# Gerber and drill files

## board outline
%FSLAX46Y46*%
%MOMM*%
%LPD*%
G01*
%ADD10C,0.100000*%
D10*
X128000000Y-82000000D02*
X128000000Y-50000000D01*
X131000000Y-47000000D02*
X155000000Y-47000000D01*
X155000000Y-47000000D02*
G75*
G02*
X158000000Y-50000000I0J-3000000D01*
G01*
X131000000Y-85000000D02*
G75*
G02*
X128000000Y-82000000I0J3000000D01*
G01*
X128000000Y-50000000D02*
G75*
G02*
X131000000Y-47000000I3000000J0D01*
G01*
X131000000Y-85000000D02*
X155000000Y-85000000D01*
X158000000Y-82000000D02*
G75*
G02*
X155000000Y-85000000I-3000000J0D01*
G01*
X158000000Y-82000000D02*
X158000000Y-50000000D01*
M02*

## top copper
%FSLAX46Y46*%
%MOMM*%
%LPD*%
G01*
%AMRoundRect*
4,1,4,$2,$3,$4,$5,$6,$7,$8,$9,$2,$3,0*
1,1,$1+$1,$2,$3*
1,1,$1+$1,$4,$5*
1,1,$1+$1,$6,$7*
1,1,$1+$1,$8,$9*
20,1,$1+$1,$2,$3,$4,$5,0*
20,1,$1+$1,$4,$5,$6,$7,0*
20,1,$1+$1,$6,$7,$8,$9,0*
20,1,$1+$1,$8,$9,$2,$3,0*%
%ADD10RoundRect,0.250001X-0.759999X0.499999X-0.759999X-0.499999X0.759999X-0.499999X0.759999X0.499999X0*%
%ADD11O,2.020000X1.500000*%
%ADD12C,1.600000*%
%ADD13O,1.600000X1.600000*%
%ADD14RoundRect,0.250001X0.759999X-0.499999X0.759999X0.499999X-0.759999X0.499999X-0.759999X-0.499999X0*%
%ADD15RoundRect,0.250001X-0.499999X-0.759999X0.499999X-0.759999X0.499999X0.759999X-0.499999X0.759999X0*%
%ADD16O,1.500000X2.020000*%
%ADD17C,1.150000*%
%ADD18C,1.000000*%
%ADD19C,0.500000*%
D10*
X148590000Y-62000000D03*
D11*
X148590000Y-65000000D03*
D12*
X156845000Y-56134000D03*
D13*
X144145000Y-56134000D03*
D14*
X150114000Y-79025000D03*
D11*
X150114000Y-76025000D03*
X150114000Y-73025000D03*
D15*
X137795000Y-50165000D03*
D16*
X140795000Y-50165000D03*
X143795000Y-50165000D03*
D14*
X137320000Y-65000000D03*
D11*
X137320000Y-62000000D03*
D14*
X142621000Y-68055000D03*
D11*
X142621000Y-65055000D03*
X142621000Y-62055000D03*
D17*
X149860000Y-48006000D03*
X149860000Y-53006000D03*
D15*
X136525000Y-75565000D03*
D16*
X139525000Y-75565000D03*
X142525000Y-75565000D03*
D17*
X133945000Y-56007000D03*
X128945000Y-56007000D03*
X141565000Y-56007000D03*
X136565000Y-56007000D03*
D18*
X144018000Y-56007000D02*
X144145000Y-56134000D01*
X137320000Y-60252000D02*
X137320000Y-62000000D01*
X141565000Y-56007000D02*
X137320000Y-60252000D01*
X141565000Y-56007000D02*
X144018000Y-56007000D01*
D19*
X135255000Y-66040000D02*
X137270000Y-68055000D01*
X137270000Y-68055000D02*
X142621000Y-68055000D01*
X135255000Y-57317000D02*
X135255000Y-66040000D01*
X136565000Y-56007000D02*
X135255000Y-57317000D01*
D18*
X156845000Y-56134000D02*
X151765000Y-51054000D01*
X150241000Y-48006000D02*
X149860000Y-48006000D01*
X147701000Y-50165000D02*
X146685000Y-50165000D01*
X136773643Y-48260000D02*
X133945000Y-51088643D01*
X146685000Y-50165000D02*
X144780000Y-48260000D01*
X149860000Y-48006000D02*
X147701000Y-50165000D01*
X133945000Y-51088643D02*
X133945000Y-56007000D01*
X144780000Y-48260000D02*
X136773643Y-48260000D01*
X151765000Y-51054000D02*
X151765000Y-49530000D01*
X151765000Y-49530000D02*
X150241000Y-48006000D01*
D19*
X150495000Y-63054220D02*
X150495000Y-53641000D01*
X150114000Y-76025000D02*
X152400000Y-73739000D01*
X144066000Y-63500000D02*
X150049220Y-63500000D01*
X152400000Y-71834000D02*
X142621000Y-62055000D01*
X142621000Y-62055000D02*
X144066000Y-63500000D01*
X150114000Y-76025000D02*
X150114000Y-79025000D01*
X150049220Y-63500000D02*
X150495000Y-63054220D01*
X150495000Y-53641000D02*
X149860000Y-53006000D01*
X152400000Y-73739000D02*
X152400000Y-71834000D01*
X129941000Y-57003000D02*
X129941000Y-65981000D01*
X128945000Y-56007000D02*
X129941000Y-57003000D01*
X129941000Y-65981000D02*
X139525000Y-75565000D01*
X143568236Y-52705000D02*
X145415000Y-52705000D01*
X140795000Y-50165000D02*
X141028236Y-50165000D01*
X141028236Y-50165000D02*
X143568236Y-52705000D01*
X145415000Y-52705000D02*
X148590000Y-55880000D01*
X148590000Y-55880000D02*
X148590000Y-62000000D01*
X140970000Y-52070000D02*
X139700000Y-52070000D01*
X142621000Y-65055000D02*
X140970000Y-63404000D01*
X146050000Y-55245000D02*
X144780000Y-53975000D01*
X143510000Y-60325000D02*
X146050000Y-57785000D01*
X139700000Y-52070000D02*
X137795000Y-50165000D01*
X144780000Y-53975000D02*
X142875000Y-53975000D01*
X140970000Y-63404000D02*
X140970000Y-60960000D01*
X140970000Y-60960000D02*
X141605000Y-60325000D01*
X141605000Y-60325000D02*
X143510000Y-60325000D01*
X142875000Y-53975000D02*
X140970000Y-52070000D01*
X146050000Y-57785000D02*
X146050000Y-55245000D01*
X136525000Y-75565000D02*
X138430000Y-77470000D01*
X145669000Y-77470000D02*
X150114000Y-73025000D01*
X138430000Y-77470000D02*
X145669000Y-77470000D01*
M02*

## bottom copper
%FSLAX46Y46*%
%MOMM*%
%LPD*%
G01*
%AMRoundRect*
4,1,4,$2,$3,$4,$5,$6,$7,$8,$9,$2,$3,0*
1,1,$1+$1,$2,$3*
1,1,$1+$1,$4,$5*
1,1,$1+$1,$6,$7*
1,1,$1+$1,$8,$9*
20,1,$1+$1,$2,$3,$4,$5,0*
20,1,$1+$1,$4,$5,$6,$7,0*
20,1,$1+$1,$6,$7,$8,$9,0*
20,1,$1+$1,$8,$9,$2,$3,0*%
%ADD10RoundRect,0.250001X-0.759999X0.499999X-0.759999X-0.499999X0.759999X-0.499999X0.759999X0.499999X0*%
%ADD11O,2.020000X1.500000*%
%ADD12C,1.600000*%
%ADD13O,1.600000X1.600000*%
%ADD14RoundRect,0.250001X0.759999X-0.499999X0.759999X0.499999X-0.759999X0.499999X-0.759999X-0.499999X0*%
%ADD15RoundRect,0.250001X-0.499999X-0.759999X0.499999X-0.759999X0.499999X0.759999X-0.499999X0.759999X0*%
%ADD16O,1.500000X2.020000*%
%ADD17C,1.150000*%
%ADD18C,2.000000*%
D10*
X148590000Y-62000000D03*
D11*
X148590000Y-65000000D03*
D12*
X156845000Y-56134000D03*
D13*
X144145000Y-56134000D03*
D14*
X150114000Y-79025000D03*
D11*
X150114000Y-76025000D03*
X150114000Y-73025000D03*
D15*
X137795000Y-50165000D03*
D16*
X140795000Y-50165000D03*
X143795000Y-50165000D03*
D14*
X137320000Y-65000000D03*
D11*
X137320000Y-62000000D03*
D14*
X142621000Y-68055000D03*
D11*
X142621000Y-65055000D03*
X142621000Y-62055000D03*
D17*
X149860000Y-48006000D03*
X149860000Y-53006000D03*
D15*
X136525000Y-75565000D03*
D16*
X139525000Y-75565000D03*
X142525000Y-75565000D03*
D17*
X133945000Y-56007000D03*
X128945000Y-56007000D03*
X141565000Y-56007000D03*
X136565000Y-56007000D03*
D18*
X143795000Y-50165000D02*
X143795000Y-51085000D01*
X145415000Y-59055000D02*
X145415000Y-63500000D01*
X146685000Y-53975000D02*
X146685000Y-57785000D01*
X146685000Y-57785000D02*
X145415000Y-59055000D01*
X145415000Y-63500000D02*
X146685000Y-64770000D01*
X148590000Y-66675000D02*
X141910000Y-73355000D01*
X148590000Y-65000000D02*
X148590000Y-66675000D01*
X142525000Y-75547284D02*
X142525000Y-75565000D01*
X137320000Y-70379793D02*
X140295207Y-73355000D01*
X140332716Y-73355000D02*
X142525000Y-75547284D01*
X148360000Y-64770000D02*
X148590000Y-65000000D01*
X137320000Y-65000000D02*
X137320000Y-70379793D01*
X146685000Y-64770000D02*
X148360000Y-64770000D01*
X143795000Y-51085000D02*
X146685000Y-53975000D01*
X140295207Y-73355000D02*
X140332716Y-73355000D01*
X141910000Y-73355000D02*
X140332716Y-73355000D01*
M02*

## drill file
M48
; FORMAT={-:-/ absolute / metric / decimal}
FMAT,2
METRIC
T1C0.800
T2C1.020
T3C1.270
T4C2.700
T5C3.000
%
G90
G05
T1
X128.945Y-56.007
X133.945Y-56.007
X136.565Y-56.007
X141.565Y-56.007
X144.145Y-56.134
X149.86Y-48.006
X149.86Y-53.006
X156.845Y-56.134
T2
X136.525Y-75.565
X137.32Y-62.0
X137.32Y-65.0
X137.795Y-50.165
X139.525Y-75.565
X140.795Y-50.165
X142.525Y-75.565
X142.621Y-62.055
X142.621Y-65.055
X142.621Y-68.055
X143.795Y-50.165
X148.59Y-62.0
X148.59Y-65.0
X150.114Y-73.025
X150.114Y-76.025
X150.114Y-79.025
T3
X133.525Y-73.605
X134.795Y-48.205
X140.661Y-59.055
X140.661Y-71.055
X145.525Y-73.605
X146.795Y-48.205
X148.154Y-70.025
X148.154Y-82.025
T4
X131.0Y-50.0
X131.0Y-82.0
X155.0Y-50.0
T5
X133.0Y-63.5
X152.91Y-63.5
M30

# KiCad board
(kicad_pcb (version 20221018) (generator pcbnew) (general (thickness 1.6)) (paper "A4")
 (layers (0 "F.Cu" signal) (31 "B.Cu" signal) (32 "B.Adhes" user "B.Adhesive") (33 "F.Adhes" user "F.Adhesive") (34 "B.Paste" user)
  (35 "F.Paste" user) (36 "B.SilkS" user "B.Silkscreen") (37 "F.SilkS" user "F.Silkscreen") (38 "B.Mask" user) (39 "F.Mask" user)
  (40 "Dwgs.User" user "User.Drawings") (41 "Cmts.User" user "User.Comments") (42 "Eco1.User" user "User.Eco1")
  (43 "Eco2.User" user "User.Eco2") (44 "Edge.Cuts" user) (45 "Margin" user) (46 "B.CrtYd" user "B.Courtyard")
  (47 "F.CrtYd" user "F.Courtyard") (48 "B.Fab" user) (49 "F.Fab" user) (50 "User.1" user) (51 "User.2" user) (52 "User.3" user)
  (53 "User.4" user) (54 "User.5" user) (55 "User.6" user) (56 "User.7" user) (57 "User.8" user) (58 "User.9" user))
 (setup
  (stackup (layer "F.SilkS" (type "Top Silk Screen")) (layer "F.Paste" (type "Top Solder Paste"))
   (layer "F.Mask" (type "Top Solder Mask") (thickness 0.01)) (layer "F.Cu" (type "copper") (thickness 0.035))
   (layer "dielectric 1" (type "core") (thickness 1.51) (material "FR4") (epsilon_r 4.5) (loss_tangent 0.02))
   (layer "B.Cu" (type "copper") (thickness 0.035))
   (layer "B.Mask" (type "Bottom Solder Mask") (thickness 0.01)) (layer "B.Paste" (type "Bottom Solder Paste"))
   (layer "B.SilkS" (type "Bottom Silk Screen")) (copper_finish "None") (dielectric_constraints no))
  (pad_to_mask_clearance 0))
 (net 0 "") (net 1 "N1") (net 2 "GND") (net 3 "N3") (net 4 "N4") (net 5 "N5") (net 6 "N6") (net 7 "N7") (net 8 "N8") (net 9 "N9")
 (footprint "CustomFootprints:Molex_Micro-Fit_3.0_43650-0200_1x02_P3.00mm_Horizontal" (layer "F.Cu") (at 148.59 62 -90)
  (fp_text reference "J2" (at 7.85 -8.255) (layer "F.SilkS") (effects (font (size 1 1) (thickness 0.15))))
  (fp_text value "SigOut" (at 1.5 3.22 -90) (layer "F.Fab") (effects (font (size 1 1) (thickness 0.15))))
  (pad "" np_thru_hole circle (at 1.5 -4.32 270) (size 3 3) (drill 3) (layers "*.Cu" "*.Mask"))
  (pad "1" thru_hole roundrect (at 0 0 270) (size 1.5 2.02) (drill 1.02) (layers "*.Cu" "*.Mask") (roundrect_rratio 0.166667) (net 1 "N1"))
  (pad "2" thru_hole oval (at 3 0 270) (size 1.5 2.02) (drill 1.02) (layers "*.Cu" "*.Mask") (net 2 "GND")))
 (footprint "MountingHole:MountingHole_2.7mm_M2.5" (layer "F.Cu") (at 131 50)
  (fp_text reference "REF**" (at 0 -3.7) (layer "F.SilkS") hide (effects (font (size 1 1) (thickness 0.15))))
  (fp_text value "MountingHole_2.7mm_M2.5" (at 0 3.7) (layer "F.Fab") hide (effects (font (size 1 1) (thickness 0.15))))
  (pad "" np_thru_hole circle (at 0 0) (size 2.7 2.7) (drill 2.7) (layers "*.Cu" "*.Mask")))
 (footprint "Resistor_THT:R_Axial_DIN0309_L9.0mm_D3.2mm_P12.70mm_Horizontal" (layer "F.Cu") (at 156.845 56.134 180)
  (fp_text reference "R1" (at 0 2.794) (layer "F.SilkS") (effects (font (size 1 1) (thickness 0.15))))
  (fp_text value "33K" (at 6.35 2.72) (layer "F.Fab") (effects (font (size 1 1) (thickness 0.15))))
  (pad "1" thru_hole circle (at 0 0 180) (size 1.6 1.6) (drill 0.8) (layers "*.Cu" "*.Mask") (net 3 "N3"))
  (pad "2" thru_hole oval (at 12.7 0 180) (size 1.6 1.6) (drill 0.8) (layers "*.Cu" "*.Mask") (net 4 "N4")))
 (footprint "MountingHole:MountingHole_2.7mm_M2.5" (layer "F.Cu") (at 155 50)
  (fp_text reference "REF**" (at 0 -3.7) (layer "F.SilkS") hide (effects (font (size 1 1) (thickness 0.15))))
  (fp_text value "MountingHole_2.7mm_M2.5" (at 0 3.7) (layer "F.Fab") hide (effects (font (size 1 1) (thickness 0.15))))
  (pad "" np_thru_hole circle (at 0 0) (size 2.7 2.7) (drill 2.7) (layers "*.Cu" "*.Mask")))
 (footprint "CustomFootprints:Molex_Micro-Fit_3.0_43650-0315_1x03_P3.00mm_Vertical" (layer "F.Cu") (at 150.114 79.025 90)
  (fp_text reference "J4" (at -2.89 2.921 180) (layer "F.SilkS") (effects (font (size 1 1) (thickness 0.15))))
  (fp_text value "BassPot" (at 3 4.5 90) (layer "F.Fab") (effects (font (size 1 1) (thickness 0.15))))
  (pad "" np_thru_hole circle (at -3 -1.96 90) (size 1.27 1.27) (drill 1.27) (layers "*.Cu" "*.Mask"))
  (pad "" np_thru_hole circle (at 9 -1.96 90) (size 1.27 1.27) (drill 1.27) (layers "*.Cu" "*.Mask"))
  (pad "1" thru_hole roundrect (at 0 0 90) (size 1.5 2.02) (drill 1.02) (layers "*.Cu" "*.Mask") (roundrect_rratio 0.166667) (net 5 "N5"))
  (pad "2" thru_hole oval (at 3 0 90) (size 1.5 2.02) (drill 1.02) (layers "*.Cu" "*.Mask") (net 5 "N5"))
  (pad "3" thru_hole oval (at 6 0 90) (size 1.5 2.02) (drill 1.02) (layers "*.Cu" "*.Mask") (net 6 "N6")))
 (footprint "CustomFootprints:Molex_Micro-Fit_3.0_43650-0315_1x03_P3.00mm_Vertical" (layer "F.Cu") (at 137.795 50.165)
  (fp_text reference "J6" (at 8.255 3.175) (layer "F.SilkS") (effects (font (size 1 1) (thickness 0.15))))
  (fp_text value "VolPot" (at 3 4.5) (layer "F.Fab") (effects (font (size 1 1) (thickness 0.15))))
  (pad "" np_thru_hole circle (at -3 -1.96) (size 1.27 1.27) (drill 1.27) (layers "*.Cu" "*.Mask"))
  (pad "" np_thru_hole circle (at 9 -1.96) (size 1.27 1.27) (drill 1.27) (layers "*.Cu" "*.Mask"))
  (pad "1" thru_hole roundrect (at 0 0) (size 1.5 2.02) (drill 1.02) (layers "*.Cu" "*.Mask") (roundrect_rratio 0.166667) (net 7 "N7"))
  (pad "2" thru_hole oval (at 3 0) (size 1.5 2.02) (drill 1.02) (layers "*.Cu" "*.Mask") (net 1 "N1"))
  (pad "3" thru_hole oval (at 6 0) (size 1.5 2.02) (drill 1.02) (layers "*.Cu" "*.Mask") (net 2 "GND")))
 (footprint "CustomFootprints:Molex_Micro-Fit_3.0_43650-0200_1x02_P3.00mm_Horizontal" (layer "F.Cu") (at 137.32 65 90)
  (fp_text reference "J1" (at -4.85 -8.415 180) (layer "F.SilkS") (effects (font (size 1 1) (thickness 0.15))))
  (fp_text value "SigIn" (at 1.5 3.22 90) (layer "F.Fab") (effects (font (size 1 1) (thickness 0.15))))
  (pad "" np_thru_hole circle (at 1.5 -4.32 90) (size 3 3) (drill 3) (layers "*.Cu" "*.Mask"))
  (pad "1" thru_hole roundrect (at 0 0 90) (size 1.5 2.02) (drill 1.02) (layers "*.Cu" "*.Mask") (roundrect_rratio 0.166667) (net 2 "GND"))
  (pad "2" thru_hole oval (at 3 0 90) (size 1.5 2.02) (drill 1.02) (layers "*.Cu" "*.Mask") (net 4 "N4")))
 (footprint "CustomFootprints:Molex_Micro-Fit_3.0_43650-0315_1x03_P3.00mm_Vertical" (layer "F.Cu") (at 142.621 68.055 90)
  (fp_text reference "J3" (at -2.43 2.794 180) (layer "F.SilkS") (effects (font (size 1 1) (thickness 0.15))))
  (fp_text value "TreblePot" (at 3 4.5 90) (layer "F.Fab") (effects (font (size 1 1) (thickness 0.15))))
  (pad "" np_thru_hole circle (at -3 -1.96 90) (size 1.27 1.27) (drill 1.27) (layers "*.Cu" "*.Mask"))
  (pad "" np_thru_hole circle (at 9 -1.96 90) (size 1.27 1.27) (drill 1.27) (layers "*.Cu" "*.Mask"))
  (pad "1" thru_hole roundrect (at 0 0 90) (size 1.5 2.02) (drill 1.02) (layers "*.Cu" "*.Mask") (roundrect_rratio 0.166667) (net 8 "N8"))
  (pad "2" thru_hole oval (at 3 0 90) (size 1.5 2.02) (drill 1.02) (layers "*.Cu" "*.Mask") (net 7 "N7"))
  (pad "3" thru_hole oval (at 6 0 90) (size 1.5 2.02) (drill 1.02) (layers "*.Cu" "*.Mask") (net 5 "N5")))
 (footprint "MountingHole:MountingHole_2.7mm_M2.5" (layer "F.Cu") (at 131 82)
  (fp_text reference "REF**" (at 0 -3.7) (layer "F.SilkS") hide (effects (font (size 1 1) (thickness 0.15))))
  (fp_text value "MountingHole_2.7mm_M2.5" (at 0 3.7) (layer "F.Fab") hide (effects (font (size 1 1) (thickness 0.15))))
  (pad "" np_thru_hole circle (at 0 0) (size 2.7 2.7) (drill 2.7) (layers "*.Cu" "*.Mask")))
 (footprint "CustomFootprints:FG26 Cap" (layer "F.Cu") (at 149.86 50.506 -90)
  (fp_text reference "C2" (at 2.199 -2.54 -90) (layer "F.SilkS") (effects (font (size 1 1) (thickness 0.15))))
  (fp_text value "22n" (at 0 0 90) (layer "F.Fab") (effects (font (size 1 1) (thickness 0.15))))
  (pad "1" thru_hole circle (at -2.5 0 270) (size 1.15 1.15) (drill 0.8) (layers "*.Cu" "*.Mask") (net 3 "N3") (solder_mask_margin 0.102))
  (pad "2" thru_hole circle (at 2.5 0 270) (size 1.15 1.15) (drill 0.8) (layers "*.Cu" "*.Mask") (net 5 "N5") (solder_mask_margin 0.102)))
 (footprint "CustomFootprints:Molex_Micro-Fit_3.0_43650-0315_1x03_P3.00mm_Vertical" (layer "F.Cu") (at 136.525 75.565)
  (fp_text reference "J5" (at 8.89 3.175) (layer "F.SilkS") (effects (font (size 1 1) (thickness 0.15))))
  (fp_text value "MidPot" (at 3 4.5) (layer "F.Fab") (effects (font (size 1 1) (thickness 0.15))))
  (pad "" np_thru_hole circle (at -3 -1.96) (size 1.27 1.27) (drill 1.27) (layers "*.Cu" "*.Mask"))
  (pad "" np_thru_hole circle (at 9 -1.96) (size 1.27 1.27) (drill 1.27) (layers "*.Cu" "*.Mask"))
  (pad "1" thru_hole roundrect (at 0 0) (size 1.5 2.02) (drill 1.02) (layers "*.Cu" "*.Mask") (roundrect_rratio 0.166667) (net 6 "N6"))
  (pad "2" thru_hole oval (at 3 0) (size 1.5 2.02) (drill 1.02) (layers "*.Cu" "*.Mask") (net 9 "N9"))
  (pad "3" thru_hole oval (at 6 0) (size 1.5 2.02) (drill 1.02) (layers "*.Cu" "*.Mask") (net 2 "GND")))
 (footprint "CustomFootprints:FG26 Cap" (layer "F.Cu") (at 131.445 56.007 180)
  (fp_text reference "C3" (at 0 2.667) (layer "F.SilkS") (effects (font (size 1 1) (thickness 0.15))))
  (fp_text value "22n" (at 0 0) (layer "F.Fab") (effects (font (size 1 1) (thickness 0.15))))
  (pad "1" thru_hole circle (at -2.5 0 180) (size 1.15 1.15) (drill 0.8) (layers "*.Cu" "*.Mask") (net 3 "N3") (solder_mask_margin 0.102))
  (pad "2" thru_hole circle (at 2.5 0 180) (size 1.15 1.15) (drill 0.8) (layers "*.Cu" "*.Mask") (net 9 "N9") (solder_mask_margin 0.102)))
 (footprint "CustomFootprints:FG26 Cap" (layer "F.Cu") (at 139.065 56.007 180)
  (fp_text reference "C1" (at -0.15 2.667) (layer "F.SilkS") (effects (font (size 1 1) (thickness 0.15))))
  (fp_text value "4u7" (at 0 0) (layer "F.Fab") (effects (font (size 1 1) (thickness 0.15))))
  (pad "1" thru_hole circle (at -2.5 0 180) (size 1.15 1.15) (drill 0.8) (layers "*.Cu" "*.Mask") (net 4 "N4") (solder_mask_margin 0.102))
  (pad "2" thru_hole circle (at 2.5 0 180) (size 1.15 1.15) (drill 0.8) (layers "*.Cu" "*.Mask") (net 8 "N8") (solder_mask_margin 0.102)))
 (gr_line (start 128 82) (end 128 50) (stroke (width 0.1) (type default)) (layer "Edge.Cuts"))
 (gr_line (start 131 47) (end 155 47) (stroke (width 0.1) (type default)) (layer "Edge.Cuts"))
 (gr_arc (start 155 47) (mid 157.12132 47.87868) (end 158 50) (stroke (width 0.1) (type default)) (layer "Edge.Cuts"))
 (gr_arc (start 131 85) (mid 128.87868 84.12132) (end 128 82) (stroke (width 0.1) (type default)) (layer "Edge.Cuts"))
 (gr_arc (start 128 50) (mid 128.87868 47.87868) (end 131 47) (stroke (width 0.1) (type default)) (layer "Edge.Cuts"))
 (gr_line (start 131 85) (end 155 85) (stroke (width 0.1) (type default)) (layer "Edge.Cuts"))
 (gr_arc (start 158 82) (mid 157.12132 84.12132) (end 155 85) (stroke (width 0.1) (type default)) (layer "Edge.Cuts"))
 (gr_line (start 158 82) (end 158 50) (stroke (width 0.1) (type default)) (layer "Edge.Cuts"))
 (segment (start 144.018 56.007) (end 144.145 56.134) (width 1) (layer "F.Cu") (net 4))
 (segment (start 137.32 60.252) (end 137.32 62) (width 1) (layer "F.Cu") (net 4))
 (segment (start 141.565 56.007) (end 137.32 60.252) (width 1) (layer "F.Cu") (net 4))
 (segment (start 141.565 56.007) (end 144.018 56.007) (width 1) (layer "F.Cu") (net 4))
 (segment (start 135.255 66.04) (end 137.27 68.055) (width 0.5) (layer "F.Cu") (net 8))
 (segment (start 137.27 68.055) (end 142.621 68.055) (width 0.5) (layer "F.Cu") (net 8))
 (segment (start 135.255 57.317) (end 135.255 66.04) (width 0.5) (layer "F.Cu") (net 8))
 (segment (start 136.565 56.007) (end 135.255 57.317) (width 0.5) (layer "F.Cu") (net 8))
 (segment (start 156.845 56.134) (end 151.765 51.054) (width 1) (layer "F.Cu") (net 3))
 (segment (start 150.241 48.006) (end 149.86 48.006) (width 1) (layer "F.Cu") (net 3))
 (segment (start 147.701 50.165) (end 146.685 50.165) (width 1) (layer "F.Cu") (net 3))
 (segment (start 136.773643 48.26) (end 133.945 51.088643) (width 1) (layer "F.Cu") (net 3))
 (segment (start 146.685 50.165) (end 144.78 48.26) (width 1) (layer "F.Cu") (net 3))
 (segment (start 149.86 48.006) (end 147.701 50.165) (width 1) (layer "F.Cu") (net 3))
 (segment (start 133.945 51.088643) (end 133.945 56.007) (width 1) (layer "F.Cu") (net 3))
 (segment (start 144.78 48.26) (end 136.773643 48.26) (width 1) (layer "F.Cu") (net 3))
 (segment (start 151.765 51.054) (end 151.765 49.53) (width 1) (layer "F.Cu") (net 3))
 (segment (start 151.765 49.53) (end 150.241 48.006) (width 1) (layer "F.Cu") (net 3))
 (segment (start 150.495 63.05422) (end 150.495 53.641) (width 0.5) (layer "F.Cu") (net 5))
 (segment (start 150.114 76.025) (end 152.4 73.739) (width 0.5) (layer "F.Cu") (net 5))
 (segment (start 144.066 63.5) (end 150.04922 63.5) (width 0.5) (layer "F.Cu") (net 5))
 (segment (start 152.4 71.834) (end 142.621 62.055) (width 0.5) (layer "F.Cu") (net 5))
 (segment (start 142.621 62.055) (end 144.066 63.5) (width 0.5) (layer "F.Cu") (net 5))
 (segment (start 150.114 76.025) (end 150.114 79.025) (width 0.5) (layer "F.Cu") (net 5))
 (segment (start 150.04922 63.5) (end 150.495 63.05422) (width 0.5) (layer "F.Cu") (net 5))
 (segment (start 150.495 53.641) (end 149.86 53.006) (width 0.5) (layer "F.Cu") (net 5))
 (segment (start 152.4 73.739) (end 152.4 71.834) (width 0.5) (layer "F.Cu") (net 5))
 (segment (start 129.941 57.003) (end 129.941 65.981) (width 0.5) (layer "F.Cu") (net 9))
 (segment (start 128.945 56.007) (end 129.941 57.003) (width 0.5) (layer "F.Cu") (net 9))
 (segment (start 129.941 65.981) (end 139.525 75.565) (width 0.5) (layer "F.Cu") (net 9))
 (segment (start 143.795 50.165) (end 143.795 51.085) (width 2) (layer "B.Cu") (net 2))
 (segment (start 145.415 59.055) (end 145.415 63.5) (width 2) (layer "B.Cu") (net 2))
 (segment (start 146.685 53.975) (end 146.685 57.785) (width 2) (layer "B.Cu") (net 2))
 (segment (start 146.685 57.785) (end 145.415 59.055) (width 2) (layer "B.Cu") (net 2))
 (segment (start 145.415 63.5) (end 146.685 64.77) (width 2) (layer "B.Cu") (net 2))
 (segment (start 148.59 66.675) (end 141.91 73.355) (width 2) (layer "B.Cu") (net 2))
 (segment (start 148.59 65) (end 148.59 66.675) (width 2) (layer "B.Cu") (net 2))
 (segment (start 142.525 75.547284) (end 142.525 75.565) (width 2) (layer "B.Cu") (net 2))
 (segment (start 137.32 70.379793) (end 140.295207 73.355) (width 2) (layer "B.Cu") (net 2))
 (segment (start 140.332716 73.355) (end 142.525 75.547284) (width 2) (layer "B.Cu") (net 2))
 (segment (start 148.36 64.77) (end 148.59 65) (width 2) (layer "B.Cu") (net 2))
 (segment (start 137.32 65) (end 137.32 70.379793) (width 2) (layer "B.Cu") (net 2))
 (segment (start 146.685 64.77) (end 148.36 64.77) (width 2) (layer "B.Cu") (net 2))
 (segment (start 143.795 51.085) (end 146.685 53.975) (width 2) (layer "B.Cu") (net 2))
 (segment (start 140.295207 73.355) (end 140.332716 73.355) (width 2) (layer "B.Cu") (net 2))
 (segment (start 141.91 73.355) (end 140.332716 73.355) (width 2) (layer "B.Cu") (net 2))
 (segment (start 143.568236 52.705) (end 145.415 52.705) (width 0.5) (layer "F.Cu") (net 1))
 (segment (start 140.795 50.165) (end 141.028236 50.165) (width 0.5) (layer "F.Cu") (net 1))
 (segment (start 141.028236 50.165) (end 143.568236 52.705) (width 0.5) (layer "F.Cu") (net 1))
 (segment (start 145.415 52.705) (end 148.59 55.88) (width 0.5) (layer "F.Cu") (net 1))
 (segment (start 148.59 55.88) (end 148.59 62) (width 0.5) (layer "F.Cu") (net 1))
 (segment (start 140.97 52.07) (end 139.7 52.07) (width 0.5) (layer "F.Cu") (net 7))
 (segment (start 142.621 65.055) (end 140.97 63.404) (width 0.5) (layer "F.Cu") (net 7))
 (segment (start 146.05 55.245) (end 144.78 53.975) (width 0.5) (layer "F.Cu") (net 7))
 (segment (start 143.51 60.325) (end 146.05 57.785) (width 0.5) (layer "F.Cu") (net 7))
 (segment (start 139.7 52.07) (end 137.795 50.165) (width 0.5) (layer "F.Cu") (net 7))
 (segment (start 144.78 53.975) (end 142.875 53.975) (width 0.5) (layer "F.Cu") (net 7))
 (segment (start 140.97 63.404) (end 140.97 60.96) (width 0.5) (layer "F.Cu") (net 7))
 (segment (start 140.97 60.96) (end 141.605 60.325) (width 0.5) (layer "F.Cu") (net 7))
 (segment (start 141.605 60.325) (end 143.51 60.325) (width 0.5) (layer "F.Cu") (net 7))
 (segment (start 142.875 53.975) (end 140.97 52.07) (width 0.5) (layer "F.Cu") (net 7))
 (segment (start 146.05 57.785) (end 146.05 55.245) (width 0.5) (layer "F.Cu") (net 7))
 (segment (start 136.525 75.565) (end 138.43 77.47) (width 0.5) (layer "F.Cu") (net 6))
 (segment (start 145.669 77.47) (end 150.114 73.025) (width 0.5) (layer "F.Cu") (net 6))
 (segment (start 138.43 77.47) (end 145.669 77.47) (width 0.5) (layer "F.Cu") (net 6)))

